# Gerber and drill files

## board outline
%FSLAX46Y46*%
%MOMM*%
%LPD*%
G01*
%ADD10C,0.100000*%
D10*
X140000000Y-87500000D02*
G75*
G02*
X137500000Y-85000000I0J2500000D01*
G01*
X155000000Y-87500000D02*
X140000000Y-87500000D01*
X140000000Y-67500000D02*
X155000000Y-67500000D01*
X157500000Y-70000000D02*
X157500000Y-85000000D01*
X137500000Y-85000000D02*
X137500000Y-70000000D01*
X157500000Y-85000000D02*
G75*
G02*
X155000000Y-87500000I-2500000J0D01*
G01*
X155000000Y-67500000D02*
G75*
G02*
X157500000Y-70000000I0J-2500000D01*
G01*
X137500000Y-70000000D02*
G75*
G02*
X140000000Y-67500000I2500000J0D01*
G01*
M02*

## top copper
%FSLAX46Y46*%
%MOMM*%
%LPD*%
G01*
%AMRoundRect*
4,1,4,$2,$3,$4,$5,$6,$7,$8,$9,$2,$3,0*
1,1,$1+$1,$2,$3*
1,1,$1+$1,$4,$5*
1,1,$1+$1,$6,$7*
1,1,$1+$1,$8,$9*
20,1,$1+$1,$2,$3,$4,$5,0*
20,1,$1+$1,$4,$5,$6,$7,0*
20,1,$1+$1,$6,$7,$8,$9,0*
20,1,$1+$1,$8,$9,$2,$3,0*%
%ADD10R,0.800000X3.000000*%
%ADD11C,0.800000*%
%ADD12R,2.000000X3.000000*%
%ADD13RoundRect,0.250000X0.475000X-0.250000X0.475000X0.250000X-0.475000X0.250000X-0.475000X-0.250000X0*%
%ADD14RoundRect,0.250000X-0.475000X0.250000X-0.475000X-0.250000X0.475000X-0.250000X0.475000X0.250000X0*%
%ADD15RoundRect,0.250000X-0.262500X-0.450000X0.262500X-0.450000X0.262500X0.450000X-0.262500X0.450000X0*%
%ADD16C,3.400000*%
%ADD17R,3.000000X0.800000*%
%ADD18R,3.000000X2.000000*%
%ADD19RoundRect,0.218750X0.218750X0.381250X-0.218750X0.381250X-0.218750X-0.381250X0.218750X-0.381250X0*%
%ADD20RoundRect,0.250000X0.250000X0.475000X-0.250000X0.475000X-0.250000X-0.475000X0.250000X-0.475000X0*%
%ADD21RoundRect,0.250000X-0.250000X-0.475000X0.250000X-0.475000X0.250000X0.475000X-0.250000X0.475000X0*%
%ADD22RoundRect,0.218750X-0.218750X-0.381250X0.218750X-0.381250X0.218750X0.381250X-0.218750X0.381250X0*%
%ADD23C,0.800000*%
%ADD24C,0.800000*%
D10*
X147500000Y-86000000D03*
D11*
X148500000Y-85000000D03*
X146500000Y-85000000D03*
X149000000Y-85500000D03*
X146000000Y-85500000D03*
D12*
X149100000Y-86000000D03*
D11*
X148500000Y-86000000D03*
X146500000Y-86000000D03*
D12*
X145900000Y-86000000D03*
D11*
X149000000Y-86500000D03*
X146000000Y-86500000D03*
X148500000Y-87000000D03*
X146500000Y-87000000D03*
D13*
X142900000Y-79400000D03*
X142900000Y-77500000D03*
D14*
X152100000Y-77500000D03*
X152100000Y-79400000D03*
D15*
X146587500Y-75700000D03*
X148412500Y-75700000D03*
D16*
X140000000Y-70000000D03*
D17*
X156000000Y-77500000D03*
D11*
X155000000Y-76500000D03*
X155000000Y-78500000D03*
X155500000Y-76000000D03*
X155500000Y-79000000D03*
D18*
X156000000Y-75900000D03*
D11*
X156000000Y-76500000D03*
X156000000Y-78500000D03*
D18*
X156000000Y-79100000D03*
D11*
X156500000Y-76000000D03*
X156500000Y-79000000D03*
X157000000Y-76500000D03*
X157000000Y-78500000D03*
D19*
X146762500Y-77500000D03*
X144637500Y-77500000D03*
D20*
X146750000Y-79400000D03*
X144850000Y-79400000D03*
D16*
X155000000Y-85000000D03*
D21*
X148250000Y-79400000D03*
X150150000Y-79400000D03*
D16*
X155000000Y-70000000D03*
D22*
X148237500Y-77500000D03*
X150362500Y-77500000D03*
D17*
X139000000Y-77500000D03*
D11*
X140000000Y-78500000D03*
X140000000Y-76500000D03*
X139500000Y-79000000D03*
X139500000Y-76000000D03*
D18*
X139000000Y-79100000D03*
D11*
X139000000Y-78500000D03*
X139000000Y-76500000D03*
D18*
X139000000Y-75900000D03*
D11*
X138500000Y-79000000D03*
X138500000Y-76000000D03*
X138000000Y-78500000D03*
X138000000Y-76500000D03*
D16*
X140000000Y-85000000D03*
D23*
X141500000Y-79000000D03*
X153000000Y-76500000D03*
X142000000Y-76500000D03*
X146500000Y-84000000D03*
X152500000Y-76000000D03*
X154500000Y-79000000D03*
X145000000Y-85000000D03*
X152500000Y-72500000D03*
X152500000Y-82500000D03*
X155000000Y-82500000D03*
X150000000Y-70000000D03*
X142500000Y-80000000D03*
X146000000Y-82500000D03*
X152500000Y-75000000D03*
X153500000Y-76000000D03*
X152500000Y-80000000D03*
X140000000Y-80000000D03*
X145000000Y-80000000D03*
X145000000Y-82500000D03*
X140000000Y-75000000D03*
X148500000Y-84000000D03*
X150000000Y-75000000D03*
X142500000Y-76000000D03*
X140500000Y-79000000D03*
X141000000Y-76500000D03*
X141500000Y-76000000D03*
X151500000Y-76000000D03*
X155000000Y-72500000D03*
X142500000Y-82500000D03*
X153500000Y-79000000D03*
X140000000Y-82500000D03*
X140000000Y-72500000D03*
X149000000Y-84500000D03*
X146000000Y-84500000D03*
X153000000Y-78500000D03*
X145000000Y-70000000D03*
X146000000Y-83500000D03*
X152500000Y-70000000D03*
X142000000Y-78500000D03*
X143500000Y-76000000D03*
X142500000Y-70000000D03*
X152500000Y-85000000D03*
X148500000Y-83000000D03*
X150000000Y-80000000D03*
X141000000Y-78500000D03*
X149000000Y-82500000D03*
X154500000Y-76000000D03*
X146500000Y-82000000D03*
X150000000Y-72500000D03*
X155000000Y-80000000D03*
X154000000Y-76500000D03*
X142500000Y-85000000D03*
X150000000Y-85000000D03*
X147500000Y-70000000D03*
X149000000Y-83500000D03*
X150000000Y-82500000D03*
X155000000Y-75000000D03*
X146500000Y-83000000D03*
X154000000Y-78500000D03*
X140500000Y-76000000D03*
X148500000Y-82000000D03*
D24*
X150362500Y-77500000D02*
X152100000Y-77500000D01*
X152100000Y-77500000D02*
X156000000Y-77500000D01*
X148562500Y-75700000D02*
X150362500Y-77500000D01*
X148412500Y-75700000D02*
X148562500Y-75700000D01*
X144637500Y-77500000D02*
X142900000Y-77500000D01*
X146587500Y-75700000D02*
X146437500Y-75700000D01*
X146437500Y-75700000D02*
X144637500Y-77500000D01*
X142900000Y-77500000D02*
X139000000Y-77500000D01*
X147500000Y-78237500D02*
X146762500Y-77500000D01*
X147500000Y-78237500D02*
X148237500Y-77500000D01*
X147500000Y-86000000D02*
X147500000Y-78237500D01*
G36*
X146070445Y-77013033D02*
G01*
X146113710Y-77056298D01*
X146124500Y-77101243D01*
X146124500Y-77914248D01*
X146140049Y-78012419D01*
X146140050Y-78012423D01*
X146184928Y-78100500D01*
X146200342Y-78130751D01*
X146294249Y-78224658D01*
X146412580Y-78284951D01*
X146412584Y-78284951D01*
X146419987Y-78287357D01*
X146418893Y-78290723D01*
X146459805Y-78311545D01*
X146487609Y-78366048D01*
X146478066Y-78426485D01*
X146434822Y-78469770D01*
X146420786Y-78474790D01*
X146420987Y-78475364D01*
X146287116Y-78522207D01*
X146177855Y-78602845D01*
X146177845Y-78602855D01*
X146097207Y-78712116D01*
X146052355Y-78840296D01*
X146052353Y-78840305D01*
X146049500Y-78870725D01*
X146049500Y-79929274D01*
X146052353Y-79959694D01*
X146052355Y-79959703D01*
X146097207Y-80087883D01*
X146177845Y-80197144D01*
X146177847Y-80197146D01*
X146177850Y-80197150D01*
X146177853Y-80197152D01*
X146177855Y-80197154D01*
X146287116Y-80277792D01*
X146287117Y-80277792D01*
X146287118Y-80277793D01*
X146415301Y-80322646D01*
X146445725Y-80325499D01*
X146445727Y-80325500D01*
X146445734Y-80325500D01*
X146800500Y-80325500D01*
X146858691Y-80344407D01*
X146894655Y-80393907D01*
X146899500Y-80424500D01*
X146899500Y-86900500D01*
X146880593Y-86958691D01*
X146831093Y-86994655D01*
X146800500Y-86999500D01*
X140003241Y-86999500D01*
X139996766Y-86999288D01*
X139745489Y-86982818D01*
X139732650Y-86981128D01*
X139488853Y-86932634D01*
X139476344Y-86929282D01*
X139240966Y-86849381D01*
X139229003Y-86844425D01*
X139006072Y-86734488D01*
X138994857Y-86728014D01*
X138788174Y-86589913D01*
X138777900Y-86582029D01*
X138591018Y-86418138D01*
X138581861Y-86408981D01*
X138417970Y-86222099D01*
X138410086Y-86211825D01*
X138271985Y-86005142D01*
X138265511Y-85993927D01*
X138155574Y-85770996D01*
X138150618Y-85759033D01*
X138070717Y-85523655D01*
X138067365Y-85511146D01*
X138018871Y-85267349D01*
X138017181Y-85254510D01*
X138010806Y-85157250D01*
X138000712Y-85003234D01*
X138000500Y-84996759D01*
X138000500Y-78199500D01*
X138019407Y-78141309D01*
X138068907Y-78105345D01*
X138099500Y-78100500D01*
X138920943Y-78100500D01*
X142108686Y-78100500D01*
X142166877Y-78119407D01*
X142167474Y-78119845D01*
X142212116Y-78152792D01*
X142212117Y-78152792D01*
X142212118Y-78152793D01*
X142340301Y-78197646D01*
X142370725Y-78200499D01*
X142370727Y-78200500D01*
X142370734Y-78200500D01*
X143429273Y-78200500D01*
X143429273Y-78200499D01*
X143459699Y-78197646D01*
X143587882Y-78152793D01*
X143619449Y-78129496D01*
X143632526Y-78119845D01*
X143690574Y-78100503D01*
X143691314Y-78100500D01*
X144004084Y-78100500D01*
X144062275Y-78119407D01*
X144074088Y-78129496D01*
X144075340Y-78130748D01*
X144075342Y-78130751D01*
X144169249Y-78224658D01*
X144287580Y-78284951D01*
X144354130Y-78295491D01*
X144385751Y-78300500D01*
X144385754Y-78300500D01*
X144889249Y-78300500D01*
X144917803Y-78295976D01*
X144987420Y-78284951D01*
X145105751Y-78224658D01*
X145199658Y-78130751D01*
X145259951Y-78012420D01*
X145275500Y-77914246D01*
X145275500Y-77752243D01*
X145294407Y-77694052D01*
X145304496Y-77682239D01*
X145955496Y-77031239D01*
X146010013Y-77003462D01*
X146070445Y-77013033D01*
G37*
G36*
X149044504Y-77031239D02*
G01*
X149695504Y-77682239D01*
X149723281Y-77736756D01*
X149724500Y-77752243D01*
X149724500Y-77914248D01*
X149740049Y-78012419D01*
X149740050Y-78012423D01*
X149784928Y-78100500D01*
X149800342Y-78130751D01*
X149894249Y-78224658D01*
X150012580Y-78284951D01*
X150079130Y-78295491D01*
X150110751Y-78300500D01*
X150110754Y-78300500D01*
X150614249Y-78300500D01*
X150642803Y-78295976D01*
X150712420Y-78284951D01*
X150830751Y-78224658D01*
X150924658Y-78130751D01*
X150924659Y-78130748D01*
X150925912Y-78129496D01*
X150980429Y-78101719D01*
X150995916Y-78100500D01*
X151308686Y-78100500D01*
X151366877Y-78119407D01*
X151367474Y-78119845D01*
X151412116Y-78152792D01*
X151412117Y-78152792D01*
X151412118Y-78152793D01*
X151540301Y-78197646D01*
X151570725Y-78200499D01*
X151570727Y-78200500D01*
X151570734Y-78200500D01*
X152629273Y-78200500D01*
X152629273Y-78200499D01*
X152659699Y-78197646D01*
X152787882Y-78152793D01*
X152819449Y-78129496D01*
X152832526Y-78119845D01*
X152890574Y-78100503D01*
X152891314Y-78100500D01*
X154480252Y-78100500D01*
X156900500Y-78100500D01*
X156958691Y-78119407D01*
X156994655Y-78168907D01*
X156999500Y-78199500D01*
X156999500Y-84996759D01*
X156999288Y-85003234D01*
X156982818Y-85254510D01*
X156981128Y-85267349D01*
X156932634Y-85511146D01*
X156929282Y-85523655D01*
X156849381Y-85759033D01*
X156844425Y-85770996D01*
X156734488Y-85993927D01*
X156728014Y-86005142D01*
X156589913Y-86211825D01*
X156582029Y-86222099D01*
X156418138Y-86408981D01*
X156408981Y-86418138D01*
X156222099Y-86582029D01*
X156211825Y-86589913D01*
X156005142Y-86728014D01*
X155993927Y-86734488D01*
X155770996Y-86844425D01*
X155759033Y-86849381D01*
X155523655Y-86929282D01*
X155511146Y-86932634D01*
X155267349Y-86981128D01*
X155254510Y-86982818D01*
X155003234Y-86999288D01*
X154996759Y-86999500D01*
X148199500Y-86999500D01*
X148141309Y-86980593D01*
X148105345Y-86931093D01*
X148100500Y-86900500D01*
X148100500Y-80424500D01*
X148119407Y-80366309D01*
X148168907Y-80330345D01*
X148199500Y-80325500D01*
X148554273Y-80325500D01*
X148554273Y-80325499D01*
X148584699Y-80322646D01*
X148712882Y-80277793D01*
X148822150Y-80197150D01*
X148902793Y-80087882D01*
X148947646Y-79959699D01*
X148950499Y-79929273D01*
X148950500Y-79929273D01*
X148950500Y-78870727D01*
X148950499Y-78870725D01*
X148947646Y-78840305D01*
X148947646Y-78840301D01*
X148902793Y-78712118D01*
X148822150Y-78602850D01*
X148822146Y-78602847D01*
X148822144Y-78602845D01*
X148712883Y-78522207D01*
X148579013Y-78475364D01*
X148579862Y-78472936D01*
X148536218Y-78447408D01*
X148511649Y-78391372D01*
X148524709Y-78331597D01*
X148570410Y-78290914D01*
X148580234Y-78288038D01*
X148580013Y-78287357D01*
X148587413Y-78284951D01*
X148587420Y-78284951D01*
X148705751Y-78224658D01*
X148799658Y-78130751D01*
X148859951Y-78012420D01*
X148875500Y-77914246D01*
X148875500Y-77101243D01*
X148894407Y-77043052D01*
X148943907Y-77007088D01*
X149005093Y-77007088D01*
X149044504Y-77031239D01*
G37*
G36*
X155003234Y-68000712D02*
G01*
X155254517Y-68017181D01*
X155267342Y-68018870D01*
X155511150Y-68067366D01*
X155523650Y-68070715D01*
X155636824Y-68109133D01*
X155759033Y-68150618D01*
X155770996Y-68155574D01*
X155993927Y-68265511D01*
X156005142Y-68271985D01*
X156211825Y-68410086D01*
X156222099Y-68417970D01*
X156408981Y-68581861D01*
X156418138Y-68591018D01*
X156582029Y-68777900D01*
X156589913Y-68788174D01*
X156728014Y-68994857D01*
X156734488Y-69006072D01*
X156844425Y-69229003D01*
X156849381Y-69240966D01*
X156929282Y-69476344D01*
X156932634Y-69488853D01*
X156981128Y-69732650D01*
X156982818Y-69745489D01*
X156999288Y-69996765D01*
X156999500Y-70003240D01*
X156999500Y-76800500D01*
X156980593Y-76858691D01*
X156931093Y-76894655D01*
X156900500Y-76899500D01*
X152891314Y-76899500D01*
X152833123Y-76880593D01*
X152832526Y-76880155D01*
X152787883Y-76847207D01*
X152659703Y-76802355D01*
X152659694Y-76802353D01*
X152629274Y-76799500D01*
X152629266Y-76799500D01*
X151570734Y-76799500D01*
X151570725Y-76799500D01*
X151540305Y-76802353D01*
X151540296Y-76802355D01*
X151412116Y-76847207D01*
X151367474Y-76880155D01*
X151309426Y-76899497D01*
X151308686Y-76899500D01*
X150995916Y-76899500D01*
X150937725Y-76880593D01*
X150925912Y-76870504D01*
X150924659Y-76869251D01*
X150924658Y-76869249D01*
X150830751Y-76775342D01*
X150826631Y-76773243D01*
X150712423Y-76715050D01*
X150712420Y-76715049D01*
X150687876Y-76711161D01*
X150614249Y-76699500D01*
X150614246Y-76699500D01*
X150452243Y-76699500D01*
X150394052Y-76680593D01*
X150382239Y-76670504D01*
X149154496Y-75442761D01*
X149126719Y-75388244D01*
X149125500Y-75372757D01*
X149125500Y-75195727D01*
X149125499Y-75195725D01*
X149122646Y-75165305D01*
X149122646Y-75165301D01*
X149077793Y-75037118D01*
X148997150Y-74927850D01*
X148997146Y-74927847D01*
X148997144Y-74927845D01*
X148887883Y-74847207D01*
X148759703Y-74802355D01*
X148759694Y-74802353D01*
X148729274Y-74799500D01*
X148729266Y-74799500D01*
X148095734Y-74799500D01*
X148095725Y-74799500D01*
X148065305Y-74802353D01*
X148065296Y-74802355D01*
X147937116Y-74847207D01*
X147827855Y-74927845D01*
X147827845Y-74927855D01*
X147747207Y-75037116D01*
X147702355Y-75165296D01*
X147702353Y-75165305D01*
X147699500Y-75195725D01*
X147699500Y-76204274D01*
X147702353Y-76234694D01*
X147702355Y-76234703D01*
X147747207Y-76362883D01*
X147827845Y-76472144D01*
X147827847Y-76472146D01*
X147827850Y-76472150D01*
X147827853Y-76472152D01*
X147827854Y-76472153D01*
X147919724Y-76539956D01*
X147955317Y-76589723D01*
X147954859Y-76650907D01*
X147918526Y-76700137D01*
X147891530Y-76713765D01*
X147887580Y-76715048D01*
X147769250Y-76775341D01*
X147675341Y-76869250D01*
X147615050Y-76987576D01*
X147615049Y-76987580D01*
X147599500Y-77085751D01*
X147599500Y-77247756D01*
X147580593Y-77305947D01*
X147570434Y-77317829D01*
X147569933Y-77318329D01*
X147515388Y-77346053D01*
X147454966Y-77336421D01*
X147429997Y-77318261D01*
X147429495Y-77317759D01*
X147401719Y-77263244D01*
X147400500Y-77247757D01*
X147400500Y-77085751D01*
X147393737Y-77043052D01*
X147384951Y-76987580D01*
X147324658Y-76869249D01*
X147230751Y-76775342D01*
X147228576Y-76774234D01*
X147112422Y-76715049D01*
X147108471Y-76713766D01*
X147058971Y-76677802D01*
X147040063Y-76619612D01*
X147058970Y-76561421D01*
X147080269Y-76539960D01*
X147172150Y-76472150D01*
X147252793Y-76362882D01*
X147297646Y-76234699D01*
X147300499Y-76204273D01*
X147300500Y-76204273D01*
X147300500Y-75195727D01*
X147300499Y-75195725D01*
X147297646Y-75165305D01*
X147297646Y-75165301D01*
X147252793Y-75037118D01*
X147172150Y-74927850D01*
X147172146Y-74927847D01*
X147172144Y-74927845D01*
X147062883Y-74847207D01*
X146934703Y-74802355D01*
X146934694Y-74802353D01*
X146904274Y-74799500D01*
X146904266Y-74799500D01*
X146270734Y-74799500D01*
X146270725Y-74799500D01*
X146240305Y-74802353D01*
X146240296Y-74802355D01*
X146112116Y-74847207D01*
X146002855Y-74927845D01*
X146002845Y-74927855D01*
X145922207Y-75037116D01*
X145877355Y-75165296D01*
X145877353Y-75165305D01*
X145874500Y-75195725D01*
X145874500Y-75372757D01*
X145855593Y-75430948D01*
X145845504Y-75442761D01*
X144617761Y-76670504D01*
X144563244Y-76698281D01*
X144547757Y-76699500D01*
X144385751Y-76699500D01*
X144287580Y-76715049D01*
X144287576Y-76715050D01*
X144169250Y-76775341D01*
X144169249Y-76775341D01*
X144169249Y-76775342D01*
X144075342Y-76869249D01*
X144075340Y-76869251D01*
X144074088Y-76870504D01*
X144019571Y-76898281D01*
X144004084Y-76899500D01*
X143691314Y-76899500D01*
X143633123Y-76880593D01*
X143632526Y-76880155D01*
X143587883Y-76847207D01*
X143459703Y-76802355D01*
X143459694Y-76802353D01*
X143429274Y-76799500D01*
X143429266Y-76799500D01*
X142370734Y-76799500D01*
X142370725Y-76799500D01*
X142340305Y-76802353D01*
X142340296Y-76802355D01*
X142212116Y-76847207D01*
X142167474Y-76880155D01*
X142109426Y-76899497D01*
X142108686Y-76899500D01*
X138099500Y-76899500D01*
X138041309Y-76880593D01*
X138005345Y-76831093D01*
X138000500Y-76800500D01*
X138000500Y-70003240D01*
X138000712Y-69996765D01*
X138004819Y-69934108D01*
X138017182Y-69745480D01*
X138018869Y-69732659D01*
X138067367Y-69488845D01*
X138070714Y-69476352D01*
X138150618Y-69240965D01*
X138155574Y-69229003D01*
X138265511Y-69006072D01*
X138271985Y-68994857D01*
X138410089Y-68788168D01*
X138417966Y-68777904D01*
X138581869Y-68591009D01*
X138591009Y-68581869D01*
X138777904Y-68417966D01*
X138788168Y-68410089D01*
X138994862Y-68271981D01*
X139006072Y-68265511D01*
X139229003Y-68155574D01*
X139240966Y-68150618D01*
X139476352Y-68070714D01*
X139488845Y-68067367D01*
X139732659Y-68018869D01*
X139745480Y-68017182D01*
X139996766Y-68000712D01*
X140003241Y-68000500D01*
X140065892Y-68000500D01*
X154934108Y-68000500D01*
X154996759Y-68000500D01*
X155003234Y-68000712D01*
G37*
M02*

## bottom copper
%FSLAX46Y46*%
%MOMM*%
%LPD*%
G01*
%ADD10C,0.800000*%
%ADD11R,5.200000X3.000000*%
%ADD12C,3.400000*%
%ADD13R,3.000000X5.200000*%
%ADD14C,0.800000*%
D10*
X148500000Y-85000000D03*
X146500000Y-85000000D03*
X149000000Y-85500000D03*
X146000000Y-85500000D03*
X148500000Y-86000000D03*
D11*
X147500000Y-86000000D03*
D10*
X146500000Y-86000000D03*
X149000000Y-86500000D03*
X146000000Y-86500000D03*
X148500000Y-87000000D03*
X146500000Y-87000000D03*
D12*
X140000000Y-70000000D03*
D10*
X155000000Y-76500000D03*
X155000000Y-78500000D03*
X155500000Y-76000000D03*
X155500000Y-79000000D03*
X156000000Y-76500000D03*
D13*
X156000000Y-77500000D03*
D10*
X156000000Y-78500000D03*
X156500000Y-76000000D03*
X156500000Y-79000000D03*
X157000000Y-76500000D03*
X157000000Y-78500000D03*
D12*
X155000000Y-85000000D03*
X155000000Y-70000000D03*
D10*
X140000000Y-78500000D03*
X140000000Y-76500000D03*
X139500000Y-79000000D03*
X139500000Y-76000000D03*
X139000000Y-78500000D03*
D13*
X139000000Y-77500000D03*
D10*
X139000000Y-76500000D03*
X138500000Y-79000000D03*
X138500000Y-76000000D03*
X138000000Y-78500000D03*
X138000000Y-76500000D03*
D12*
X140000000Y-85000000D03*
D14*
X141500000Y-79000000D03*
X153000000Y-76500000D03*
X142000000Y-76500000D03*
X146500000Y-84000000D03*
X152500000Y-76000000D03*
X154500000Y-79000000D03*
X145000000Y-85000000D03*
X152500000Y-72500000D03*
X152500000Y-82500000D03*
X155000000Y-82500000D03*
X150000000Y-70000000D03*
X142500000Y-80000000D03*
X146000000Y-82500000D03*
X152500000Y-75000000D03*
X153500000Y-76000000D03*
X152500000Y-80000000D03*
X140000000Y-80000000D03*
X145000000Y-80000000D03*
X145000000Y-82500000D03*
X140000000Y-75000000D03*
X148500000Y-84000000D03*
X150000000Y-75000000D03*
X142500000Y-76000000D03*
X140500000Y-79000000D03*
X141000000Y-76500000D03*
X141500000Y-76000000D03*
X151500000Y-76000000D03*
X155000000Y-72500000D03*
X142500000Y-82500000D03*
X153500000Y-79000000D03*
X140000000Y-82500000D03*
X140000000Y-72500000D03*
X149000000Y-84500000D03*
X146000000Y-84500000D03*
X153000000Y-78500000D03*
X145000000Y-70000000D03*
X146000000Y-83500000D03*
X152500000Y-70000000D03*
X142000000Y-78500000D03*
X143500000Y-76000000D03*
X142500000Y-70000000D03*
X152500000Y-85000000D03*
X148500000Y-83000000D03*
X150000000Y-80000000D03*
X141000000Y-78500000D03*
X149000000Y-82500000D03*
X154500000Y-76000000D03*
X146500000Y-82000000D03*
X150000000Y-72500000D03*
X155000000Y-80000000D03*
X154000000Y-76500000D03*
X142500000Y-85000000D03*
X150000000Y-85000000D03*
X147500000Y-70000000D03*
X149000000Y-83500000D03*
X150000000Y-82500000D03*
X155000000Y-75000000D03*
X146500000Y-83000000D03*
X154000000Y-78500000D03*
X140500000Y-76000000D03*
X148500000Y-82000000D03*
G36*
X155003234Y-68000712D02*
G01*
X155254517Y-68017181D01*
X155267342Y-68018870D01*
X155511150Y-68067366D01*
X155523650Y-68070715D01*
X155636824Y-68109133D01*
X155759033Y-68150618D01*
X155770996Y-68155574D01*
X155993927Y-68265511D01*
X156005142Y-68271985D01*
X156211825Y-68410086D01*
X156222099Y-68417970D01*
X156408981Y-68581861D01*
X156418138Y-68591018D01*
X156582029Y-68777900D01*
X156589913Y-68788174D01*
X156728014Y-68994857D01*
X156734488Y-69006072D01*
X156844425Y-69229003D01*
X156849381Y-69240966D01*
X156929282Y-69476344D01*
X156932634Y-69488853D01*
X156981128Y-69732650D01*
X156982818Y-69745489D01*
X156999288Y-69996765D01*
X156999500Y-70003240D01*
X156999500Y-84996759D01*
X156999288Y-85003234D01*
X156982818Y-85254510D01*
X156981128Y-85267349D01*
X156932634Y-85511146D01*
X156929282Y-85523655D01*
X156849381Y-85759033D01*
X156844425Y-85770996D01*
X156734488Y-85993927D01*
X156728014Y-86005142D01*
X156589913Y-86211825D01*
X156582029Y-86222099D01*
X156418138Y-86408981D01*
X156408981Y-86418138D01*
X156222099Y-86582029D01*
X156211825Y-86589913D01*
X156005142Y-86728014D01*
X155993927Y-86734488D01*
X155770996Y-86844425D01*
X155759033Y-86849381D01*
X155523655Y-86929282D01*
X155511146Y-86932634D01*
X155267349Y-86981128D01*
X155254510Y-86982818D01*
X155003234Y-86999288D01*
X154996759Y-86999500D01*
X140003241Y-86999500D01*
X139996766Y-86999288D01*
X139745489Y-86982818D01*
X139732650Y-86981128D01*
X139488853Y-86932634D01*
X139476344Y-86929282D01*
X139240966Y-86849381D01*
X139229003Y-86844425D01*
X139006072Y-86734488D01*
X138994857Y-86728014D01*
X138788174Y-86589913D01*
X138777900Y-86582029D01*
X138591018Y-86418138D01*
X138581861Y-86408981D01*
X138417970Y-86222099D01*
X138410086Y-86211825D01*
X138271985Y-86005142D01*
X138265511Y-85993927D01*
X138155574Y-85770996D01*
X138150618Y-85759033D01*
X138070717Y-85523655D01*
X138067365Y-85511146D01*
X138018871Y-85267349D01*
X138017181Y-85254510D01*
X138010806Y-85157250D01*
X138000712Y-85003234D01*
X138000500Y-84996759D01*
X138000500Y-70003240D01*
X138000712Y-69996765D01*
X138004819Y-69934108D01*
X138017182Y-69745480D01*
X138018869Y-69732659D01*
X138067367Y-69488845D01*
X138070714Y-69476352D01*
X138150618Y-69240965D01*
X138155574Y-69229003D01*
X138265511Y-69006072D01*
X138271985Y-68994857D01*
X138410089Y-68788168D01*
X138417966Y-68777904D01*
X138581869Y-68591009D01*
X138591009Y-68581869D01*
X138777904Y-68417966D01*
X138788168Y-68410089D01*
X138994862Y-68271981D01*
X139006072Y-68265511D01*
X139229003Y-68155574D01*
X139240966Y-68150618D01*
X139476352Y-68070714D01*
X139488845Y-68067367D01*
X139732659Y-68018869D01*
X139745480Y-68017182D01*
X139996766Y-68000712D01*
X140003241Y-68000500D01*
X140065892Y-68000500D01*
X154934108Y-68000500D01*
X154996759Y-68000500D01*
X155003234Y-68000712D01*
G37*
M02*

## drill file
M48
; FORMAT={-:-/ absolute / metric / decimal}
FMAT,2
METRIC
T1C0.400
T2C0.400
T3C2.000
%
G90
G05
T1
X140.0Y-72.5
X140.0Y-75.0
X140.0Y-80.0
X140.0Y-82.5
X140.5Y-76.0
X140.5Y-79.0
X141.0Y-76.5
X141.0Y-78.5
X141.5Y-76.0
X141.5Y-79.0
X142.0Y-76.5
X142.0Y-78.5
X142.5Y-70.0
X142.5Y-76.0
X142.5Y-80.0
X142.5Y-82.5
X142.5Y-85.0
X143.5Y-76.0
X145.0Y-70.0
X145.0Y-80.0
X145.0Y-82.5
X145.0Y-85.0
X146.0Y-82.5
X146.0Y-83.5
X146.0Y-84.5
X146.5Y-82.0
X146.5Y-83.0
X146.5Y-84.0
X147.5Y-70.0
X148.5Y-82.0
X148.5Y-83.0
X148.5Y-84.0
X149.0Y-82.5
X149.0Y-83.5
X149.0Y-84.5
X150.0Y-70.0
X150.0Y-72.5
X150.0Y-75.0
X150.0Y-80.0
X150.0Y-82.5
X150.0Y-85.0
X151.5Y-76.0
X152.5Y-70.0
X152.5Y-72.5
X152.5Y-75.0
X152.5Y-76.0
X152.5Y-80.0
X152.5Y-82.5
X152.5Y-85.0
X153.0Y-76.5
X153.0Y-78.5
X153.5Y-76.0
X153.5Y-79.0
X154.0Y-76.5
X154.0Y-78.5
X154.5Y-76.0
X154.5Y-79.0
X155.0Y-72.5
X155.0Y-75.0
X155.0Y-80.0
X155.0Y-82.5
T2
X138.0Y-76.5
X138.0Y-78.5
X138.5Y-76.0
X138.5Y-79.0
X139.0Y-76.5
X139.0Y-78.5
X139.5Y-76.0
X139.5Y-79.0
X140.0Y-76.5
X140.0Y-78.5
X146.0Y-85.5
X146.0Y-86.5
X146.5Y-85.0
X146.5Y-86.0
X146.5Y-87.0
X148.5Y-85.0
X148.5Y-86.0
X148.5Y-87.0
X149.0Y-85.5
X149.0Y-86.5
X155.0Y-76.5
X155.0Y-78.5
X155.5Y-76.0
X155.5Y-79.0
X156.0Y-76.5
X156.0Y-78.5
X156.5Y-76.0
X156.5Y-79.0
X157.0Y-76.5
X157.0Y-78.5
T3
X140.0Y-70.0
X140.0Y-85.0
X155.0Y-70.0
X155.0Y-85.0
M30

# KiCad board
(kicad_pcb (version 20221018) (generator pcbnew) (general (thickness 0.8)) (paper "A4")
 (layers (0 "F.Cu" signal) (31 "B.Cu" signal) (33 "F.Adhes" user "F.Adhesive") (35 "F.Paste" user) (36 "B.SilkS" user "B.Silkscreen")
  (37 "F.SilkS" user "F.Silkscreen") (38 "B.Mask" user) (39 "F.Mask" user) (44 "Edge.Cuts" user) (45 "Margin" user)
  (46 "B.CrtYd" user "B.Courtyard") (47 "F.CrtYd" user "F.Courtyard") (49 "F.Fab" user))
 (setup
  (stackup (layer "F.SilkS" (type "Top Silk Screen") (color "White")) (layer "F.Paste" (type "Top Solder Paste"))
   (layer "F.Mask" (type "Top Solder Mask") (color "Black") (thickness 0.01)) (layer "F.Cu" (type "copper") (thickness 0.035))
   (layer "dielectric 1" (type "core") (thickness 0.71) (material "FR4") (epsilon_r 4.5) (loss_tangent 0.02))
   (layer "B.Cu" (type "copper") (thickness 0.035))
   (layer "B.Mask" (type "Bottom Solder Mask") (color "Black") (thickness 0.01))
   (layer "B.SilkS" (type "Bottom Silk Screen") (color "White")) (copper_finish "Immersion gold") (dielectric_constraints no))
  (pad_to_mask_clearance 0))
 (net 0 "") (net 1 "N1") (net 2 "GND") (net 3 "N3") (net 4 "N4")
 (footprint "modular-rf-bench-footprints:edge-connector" (layer "F.Cu") (at 147.5 87.5 -90)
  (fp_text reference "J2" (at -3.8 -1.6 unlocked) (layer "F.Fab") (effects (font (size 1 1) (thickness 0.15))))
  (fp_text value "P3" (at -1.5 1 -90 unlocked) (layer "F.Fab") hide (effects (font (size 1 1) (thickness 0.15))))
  (pad "1" smd rect (at -1.5 0 270) (size 3 0.8) (layers "F.Cu") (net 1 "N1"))
  (pad "2" thru_hole circle (at -2.5 -1 270) (size 0.8 0.8) (drill 0.4) (layers "*.Cu") (remove_unused_layers) (keep_end_layers)
   (zone_layer_connections) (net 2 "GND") (zone_connect 2))
  (pad "2" thru_hole circle (at -2.5 1 270) (size 0.8 0.8) (drill 0.4) (layers "*.Cu") (remove_unused_layers) (keep_end_layers)
   (zone_layer_connections) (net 2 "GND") (zone_connect 2))
  (pad "2" thru_hole circle (at -2 -1.5 270) (size 0.8 0.8) (drill 0.4) (layers "*.Cu") (remove_unused_layers) (keep_end_layers)
   (zone_layer_connections) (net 2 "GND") (zone_connect 2))
  (pad "2" thru_hole circle (at -2 1.5 270) (size 0.8 0.8) (drill 0.4) (layers "*.Cu") (remove_unused_layers) (keep_end_layers)
   (zone_layer_connections) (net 2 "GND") (zone_connect 2))
  (pad "2" smd rect (at -1.5 -1.6 270) (size 3 2) (layers "F.Cu") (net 2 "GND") (zone_connect 2))
  (pad "2" thru_hole circle (at -1.5 -1 270) (size 0.8 0.8) (drill 0.4) (layers "*.Cu") (remove_unused_layers) (keep_end_layers)
   (zone_layer_connections) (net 2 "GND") (zone_connect 2))
  (pad "2" smd rect (at -1.5 0 270) (size 3 5.2) (layers "B.Cu") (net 2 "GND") (zone_connect 2))
  (pad "2" thru_hole circle (at -1.5 1 270) (size 0.8 0.8) (drill 0.4) (layers "*.Cu") (remove_unused_layers) (keep_end_layers)
   (zone_layer_connections) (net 2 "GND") (zone_connect 2))
  (pad "2" smd rect (at -1.5 1.6 270) (size 3 2) (layers "F.Cu") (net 2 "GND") (zone_connect 2))
  (pad "2" thru_hole circle (at -1 -1.5 270) (size 0.8 0.8) (drill 0.4) (layers "*.Cu") (remove_unused_layers) (keep_end_layers)
   (zone_layer_connections) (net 2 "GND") (zone_connect 2))
  (pad "2" thru_hole circle (at -1 1.5 270) (size 0.8 0.8) (drill 0.4) (layers "*.Cu") (remove_unused_layers) (keep_end_layers)
   (zone_layer_connections) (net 2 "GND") (zone_connect 2))
  (pad "2" thru_hole circle (at -0.5 -1 270) (size 0.8 0.8) (drill 0.4) (layers "*.Cu") (remove_unused_layers) (keep_end_layers)
   (zone_layer_connections) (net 2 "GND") (zone_connect 2))
  (pad "2" thru_hole circle (at -0.5 1 270) (size 0.8 0.8) (drill 0.4) (layers "*.Cu") (remove_unused_layers) (keep_end_layers)
   (zone_layer_connections) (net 2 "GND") (zone_connect 2)))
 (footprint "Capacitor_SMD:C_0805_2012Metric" (layer "F.Cu") (at 142.9 78.45 90)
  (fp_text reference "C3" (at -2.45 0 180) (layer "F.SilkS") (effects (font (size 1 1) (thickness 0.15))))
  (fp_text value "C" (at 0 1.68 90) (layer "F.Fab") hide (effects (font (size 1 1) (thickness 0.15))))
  (pad "1" smd roundrect (at -0.95 0 90) (size 1 1.45) (layers "F.Cu" "F.Paste" "F.Mask") (roundrect_rratio 0.25) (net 2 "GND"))
  (pad "2" smd roundrect (at 0.95 0 90) (size 1 1.45) (layers "F.Cu" "F.Paste" "F.Mask") (roundrect_rratio 0.25) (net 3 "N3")))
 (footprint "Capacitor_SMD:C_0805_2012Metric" (layer "F.Cu") (at 152.1 78.45 -90)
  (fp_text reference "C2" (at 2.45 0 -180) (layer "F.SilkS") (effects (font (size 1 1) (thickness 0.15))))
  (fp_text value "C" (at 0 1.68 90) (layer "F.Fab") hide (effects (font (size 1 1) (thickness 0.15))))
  (pad "1" smd roundrect (at -0.95 0 270) (size 1 1.45) (layers "F.Cu" "F.Paste" "F.Mask") (roundrect_rratio 0.25) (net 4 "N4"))
  (pad "2" smd roundrect (at 0.95 0 270) (size 1 1.45) (layers "F.Cu" "F.Paste" "F.Mask") (roundrect_rratio 0.25) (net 2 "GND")))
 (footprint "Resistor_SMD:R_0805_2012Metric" (layer "F.Cu") (at 147.5 75.7)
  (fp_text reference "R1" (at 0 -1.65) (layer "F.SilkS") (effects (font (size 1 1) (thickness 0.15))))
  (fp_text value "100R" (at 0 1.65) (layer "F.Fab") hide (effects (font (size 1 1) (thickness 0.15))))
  (pad "1" smd roundrect (at -0.9125 0) (size 1.025 1.4) (layers "F.Cu" "F.Paste" "F.Mask") (roundrect_rratio 0.243902439) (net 3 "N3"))
  (pad "2" smd roundrect (at 0.9125 0) (size 1.025 1.4) (layers "F.Cu" "F.Paste" "F.Mask") (roundrect_rratio 0.243902439) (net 4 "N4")))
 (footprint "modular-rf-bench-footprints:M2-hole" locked (layer "F.Cu") (at 140 70)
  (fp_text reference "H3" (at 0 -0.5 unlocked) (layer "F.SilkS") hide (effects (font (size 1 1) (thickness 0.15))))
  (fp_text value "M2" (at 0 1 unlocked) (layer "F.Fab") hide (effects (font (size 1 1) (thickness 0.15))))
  (pad "1" thru_hole circle locked (at 0 0) (size 3.4 3.4) (drill 2) (layers "*.Cu" "*.Mask") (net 2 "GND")))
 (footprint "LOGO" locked (layer "F.Cu") (at 144.2 72.5)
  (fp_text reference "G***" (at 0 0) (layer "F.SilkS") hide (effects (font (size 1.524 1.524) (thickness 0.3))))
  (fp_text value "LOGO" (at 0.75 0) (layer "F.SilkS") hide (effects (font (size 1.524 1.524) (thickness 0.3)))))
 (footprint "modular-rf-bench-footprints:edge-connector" (layer "F.Cu") (at 157.5 77.5)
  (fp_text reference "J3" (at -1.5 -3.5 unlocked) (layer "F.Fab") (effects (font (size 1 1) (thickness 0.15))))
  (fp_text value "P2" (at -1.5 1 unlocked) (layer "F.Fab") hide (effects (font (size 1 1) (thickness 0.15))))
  (pad "1" smd rect (at -1.5 0) (size 3 0.8) (layers "F.Cu") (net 4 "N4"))
  (pad "2" thru_hole circle (at -2.5 -1) (size 0.8 0.8) (drill 0.4) (layers "*.Cu") (remove_unused_layers) (keep_end_layers)
   (zone_layer_connections) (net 2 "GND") (zone_connect 2))
  (pad "2" thru_hole circle (at -2.5 1) (size 0.8 0.8) (drill 0.4) (layers "*.Cu") (remove_unused_layers) (keep_end_layers)
   (zone_layer_connections) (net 2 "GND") (zone_connect 2))
  (pad "2" thru_hole circle (at -2 -1.5) (size 0.8 0.8) (drill 0.4) (layers "*.Cu") (remove_unused_layers) (keep_end_layers)
   (zone_layer_connections) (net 2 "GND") (zone_connect 2))
  (pad "2" thru_hole circle (at -2 1.5) (size 0.8 0.8) (drill 0.4) (layers "*.Cu") (remove_unused_layers) (keep_end_layers)
   (zone_layer_connections) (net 2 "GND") (zone_connect 2))
  (pad "2" smd rect (at -1.5 -1.6) (size 3 2) (layers "F.Cu") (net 2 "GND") (zone_connect 2))
  (pad "2" thru_hole circle (at -1.5 -1) (size 0.8 0.8) (drill 0.4) (layers "*.Cu") (remove_unused_layers) (keep_end_layers)
   (zone_layer_connections) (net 2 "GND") (zone_connect 2))
  (pad "2" smd rect (at -1.5 0) (size 3 5.2) (layers "B.Cu") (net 2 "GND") (zone_connect 2))
  (pad "2" thru_hole circle (at -1.5 1) (size 0.8 0.8) (drill 0.4) (layers "*.Cu") (remove_unused_layers) (keep_end_layers)
   (zone_layer_connections) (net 2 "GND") (zone_connect 2))
  (pad "2" smd rect (at -1.5 1.6) (size 3 2) (layers "F.Cu") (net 2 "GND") (zone_connect 2))
  (pad "2" thru_hole circle (at -1 -1.5) (size 0.8 0.8) (drill 0.4) (layers "*.Cu") (remove_unused_layers) (keep_end_layers)
   (zone_layer_connections) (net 2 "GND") (zone_connect 2))
  (pad "2" thru_hole circle (at -1 1.5) (size 0.8 0.8) (drill 0.4) (layers "*.Cu") (remove_unused_layers) (keep_end_layers)
   (zone_layer_connections) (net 2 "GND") (zone_connect 2))
  (pad "2" thru_hole circle (at -0.5 -1) (size 0.8 0.8) (drill 0.4) (layers "*.Cu") (remove_unused_layers) (keep_end_layers)
   (zone_layer_connections) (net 2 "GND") (zone_connect 2))
  (pad "2" thru_hole circle (at -0.5 1) (size 0.8 0.8) (drill 0.4) (layers "*.Cu") (remove_unused_layers) (keep_end_layers)
   (zone_layer_connections) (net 2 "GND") (zone_connect 2)))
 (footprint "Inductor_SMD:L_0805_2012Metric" (layer "F.Cu") (at 145.7 77.5 180)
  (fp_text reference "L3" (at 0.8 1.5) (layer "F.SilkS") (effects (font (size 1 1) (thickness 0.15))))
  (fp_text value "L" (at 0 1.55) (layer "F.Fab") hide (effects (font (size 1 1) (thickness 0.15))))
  (pad "1" smd roundrect (at -1.0625 0 180) (size 0.875 1.2) (layers "F.Cu" "F.Paste" "F.Mask") (roundrect_rratio 0.25) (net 1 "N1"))
  (pad "2" smd roundrect (at 1.0625 0 180) (size 0.875 1.2) (layers "F.Cu" "F.Paste" "F.Mask") (roundrect_rratio 0.25) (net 3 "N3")))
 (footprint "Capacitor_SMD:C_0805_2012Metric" (layer "F.Cu") (at 145.8 79.4 180)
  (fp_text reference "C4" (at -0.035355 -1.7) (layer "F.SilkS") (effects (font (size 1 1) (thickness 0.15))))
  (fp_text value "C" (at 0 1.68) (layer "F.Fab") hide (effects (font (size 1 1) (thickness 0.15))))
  (pad "1" smd roundrect (at -0.95 0 180) (size 1 1.45) (layers "F.Cu" "F.Paste" "F.Mask") (roundrect_rratio 0.25) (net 1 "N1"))
  (pad "2" smd roundrect (at 0.95 0 180) (size 1 1.45) (layers "F.Cu" "F.Paste" "F.Mask") (roundrect_rratio 0.25) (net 2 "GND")))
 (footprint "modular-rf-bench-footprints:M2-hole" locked (layer "F.Cu") (at 155 85)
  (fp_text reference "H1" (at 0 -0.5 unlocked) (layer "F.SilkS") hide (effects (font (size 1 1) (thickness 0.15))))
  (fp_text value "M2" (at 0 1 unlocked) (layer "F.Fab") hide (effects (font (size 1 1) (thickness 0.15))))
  (pad "1" thru_hole circle locked (at 0 0) (size 3.4 3.4) (drill 2) (layers "*.Cu" "*.Mask") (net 2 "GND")))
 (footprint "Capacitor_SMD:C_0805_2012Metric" (layer "F.Cu") (at 149.2 79.4)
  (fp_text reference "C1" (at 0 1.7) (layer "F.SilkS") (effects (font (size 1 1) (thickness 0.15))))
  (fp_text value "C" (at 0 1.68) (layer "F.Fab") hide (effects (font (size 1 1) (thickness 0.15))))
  (pad "1" smd roundrect (at -0.95 0) (size 1 1.45) (layers "F.Cu" "F.Paste" "F.Mask") (roundrect_rratio 0.25) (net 1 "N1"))
  (pad "2" smd roundrect (at 0.95 0) (size 1 1.45) (layers "F.Cu" "F.Paste" "F.Mask") (roundrect_rratio 0.25) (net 2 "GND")))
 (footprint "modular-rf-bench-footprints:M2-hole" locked (layer "F.Cu") (at 155 70)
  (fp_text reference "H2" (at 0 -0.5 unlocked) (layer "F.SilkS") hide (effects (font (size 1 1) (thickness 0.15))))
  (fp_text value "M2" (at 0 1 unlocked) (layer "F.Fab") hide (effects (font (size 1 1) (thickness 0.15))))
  (pad "1" thru_hole circle locked (at 0 0) (size 3.4 3.4) (drill 2) (layers "*.Cu" "*.Mask") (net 2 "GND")))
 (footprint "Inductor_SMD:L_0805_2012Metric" (layer "F.Cu") (at 149.3 77.5)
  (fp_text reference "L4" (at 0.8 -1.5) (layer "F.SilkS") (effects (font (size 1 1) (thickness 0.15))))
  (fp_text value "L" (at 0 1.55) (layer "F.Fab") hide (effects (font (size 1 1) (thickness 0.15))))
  (pad "1" smd roundrect (at -1.0625 0) (size 0.875 1.2) (layers "F.Cu" "F.Paste" "F.Mask") (roundrect_rratio 0.25) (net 1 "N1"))
  (pad "2" smd roundrect (at 1.0625 0) (size 0.875 1.2) (layers "F.Cu" "F.Paste" "F.Mask") (roundrect_rratio 0.25) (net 4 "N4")))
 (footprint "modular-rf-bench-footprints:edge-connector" (layer "F.Cu") (at 137.5 77.5 180)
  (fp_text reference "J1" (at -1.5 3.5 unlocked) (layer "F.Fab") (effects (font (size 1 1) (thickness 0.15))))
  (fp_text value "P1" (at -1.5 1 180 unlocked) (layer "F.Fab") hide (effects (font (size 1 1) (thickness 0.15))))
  (pad "1" smd rect (at -1.5 0 180) (size 3 0.8) (layers "F.Cu") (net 3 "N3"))
  (pad "2" thru_hole circle (at -2.5 -1 180) (size 0.8 0.8) (drill 0.4) (layers "*.Cu") (remove_unused_layers) (keep_end_layers)
   (zone_layer_connections) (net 2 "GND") (zone_connect 2))
  (pad "2" thru_hole circle (at -2.5 1 180) (size 0.8 0.8) (drill 0.4) (layers "*.Cu") (remove_unused_layers) (keep_end_layers)
   (zone_layer_connections) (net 2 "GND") (zone_connect 2))
  (pad "2" thru_hole circle (at -2 -1.5 180) (size 0.8 0.8) (drill 0.4) (layers "*.Cu") (remove_unused_layers) (keep_end_layers)
   (zone_layer_connections) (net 2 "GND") (zone_connect 2))
  (pad "2" thru_hole circle (at -2 1.5 180) (size 0.8 0.8) (drill 0.4) (layers "*.Cu") (remove_unused_layers) (keep_end_layers)
   (zone_layer_connections) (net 2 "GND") (zone_connect 2))
  (pad "2" smd rect (at -1.5 -1.6 180) (size 3 2) (layers "F.Cu") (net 2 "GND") (zone_connect 2))
  (pad "2" thru_hole circle (at -1.5 -1 180) (size 0.8 0.8) (drill 0.4) (layers "*.Cu") (remove_unused_layers) (keep_end_layers)
   (zone_layer_connections) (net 2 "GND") (zone_connect 2))
  (pad "2" smd rect (at -1.5 0 180) (size 3 5.2) (layers "B.Cu") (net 2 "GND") (zone_connect 2))
  (pad "2" thru_hole circle (at -1.5 1 180) (size 0.8 0.8) (drill 0.4) (layers "*.Cu") (remove_unused_layers) (keep_end_layers)
   (zone_layer_connections) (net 2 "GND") (zone_connect 2))
  (pad "2" smd rect (at -1.5 1.6 180) (size 3 2) (layers "F.Cu") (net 2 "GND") (zone_connect 2))
  (pad "2" thru_hole circle (at -1 -1.5 180) (size 0.8 0.8) (drill 0.4) (layers "*.Cu") (remove_unused_layers) (keep_end_layers)
   (zone_layer_connections) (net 2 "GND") (zone_connect 2))
  (pad "2" thru_hole circle (at -1 1.5 180) (size 0.8 0.8) (drill 0.4) (layers "*.Cu") (remove_unused_layers) (keep_end_layers)
   (zone_layer_connections) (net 2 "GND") (zone_connect 2))
  (pad "2" thru_hole circle (at -0.5 -1 180) (size 0.8 0.8) (drill 0.4) (layers "*.Cu") (remove_unused_layers) (keep_end_layers)
   (zone_layer_connections) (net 2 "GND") (zone_connect 2))
  (pad "2" thru_hole circle (at -0.5 1 180) (size 0.8 0.8) (drill 0.4) (layers "*.Cu") (remove_unused_layers) (keep_end_layers)
   (zone_layer_connections) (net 2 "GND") (zone_connect 2)))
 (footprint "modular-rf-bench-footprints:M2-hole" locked (layer "F.Cu") (at 140 85)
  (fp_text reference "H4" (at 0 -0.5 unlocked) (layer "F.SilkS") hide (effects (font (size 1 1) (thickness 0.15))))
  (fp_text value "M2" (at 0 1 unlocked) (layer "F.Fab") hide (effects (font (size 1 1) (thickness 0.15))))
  (pad "1" thru_hole circle locked (at 0 0) (size 3.4 3.4) (drill 2) (layers "*.Cu" "*.Mask") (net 2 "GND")))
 (gr_arc (start 140 87.5) (mid 138.232233 86.767767) (end 137.5 85) (stroke (width 0.1) (type solid)) (layer "Edge.Cuts"))
 (gr_line (start 155 87.5) (end 140 87.5) (stroke (width 0.1) (type solid)) (layer "Edge.Cuts"))
 (gr_line (start 140 67.5) (end 155 67.5) (stroke (width 0.1) (type solid)) (layer "Edge.Cuts"))
 (gr_line (start 157.5 70) (end 157.5 85) (stroke (width 0.1) (type solid)) (layer "Edge.Cuts"))
 (gr_line (start 137.5 85) (end 137.5 70) (stroke (width 0.1) (type solid)) (layer "Edge.Cuts"))
 (gr_arc (start 157.5 85) (mid 156.767767 86.767767) (end 155 87.5) (stroke (width 0.1) (type solid)) (layer "Edge.Cuts"))
 (gr_arc (start 155 67.5) (mid 156.767767 68.232233) (end 157.5 70) (stroke (width 0.1) (type solid)) (layer "Edge.Cuts"))
 (gr_arc (start 137.5 70) (mid 138.232233 68.232233) (end 140 67.5) (stroke (width 0.1) (type solid)) (layer "Edge.Cuts"))
 (via (at 141.5 79) (size 0.8) (drill 0.4) (layers "F.Cu" "B.Cu") (free) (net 2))
 (via (at 153 76.5) (size 0.8) (drill 0.4) (layers "F.Cu" "B.Cu") (free) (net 2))
 (via (at 142 76.5) (size 0.8) (drill 0.4) (layers "F.Cu" "B.Cu") (free) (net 2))
 (via (at 146.5 84) (size 0.8) (drill 0.4) (layers "F.Cu" "B.Cu") (free) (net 2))
 (via (at 152.5 76) (size 0.8) (drill 0.4) (layers "F.Cu" "B.Cu") (free) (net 2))
 (via (at 154.5 79) (size 0.8) (drill 0.4) (layers "F.Cu" "B.Cu") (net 2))
 (via (at 145 85) (size 0.8) (drill 0.4) (layers "F.Cu" "B.Cu") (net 2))
 (via (at 152.5 72.5) (size 0.8) (drill 0.4) (layers "F.Cu" "B.Cu") (free) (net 2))
 (via (at 152.5 82.5) (size 0.8) (drill 0.4) (layers "F.Cu" "B.Cu") (free) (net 2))
 (via (at 155 82.5) (size 0.8) (drill 0.4) (layers "F.Cu" "B.Cu") (free) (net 2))
 (via (at 150 70) (size 0.8) (drill 0.4) (layers "F.Cu" "B.Cu") (free) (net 2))
 (via (at 142.5 80) (size 0.8) (drill 0.4) (layers "F.Cu" "B.Cu") (free) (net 2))
 (via (at 146 82.5) (size 0.8) (drill 0.4) (layers "F.Cu" "B.Cu") (free) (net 2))
 (via (at 152.5 75) (size 0.8) (drill 0.4) (layers "F.Cu" "B.Cu") (free) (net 2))
 (via (at 153.5 76) (size 0.8) (drill 0.4) (layers "F.Cu" "B.Cu") (free) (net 2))
 (via (at 152.5 80) (size 0.8) (drill 0.4) (layers "F.Cu" "B.Cu") (free) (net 2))
 (via (at 140 80) (size 0.8) (drill 0.4) (layers "F.Cu" "B.Cu") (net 2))
 (via (at 145 80) (size 0.8) (drill 0.4) (layers "F.Cu" "B.Cu") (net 2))
 (via (at 145 82.5) (size 0.8) (drill 0.4) (layers "F.Cu" "B.Cu") (free) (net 2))
 (via (at 140 75) (size 0.8) (drill 0.4) (layers "F.Cu" "B.Cu") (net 2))
 (via (at 148.5 84) (size 0.8) (drill 0.4) (layers "F.Cu" "B.Cu") (free) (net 2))
 (via (at 150 75) (size 0.8) (drill 0.4) (layers "F.Cu" "B.Cu") (free) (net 2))
 (via (at 142.5 76) (size 0.8) (drill 0.4) (layers "F.Cu" "B.Cu") (free) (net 2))
 (via (at 140.5 79) (size 0.8) (drill 0.4) (layers "F.Cu" "B.Cu") (free) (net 2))
 (via (at 141 76.5) (size 0.8) (drill 0.4) (layers "F.Cu" "B.Cu") (free) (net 2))
 (via (at 141.5 76) (size 0.8) (drill 0.4) (layers "F.Cu" "B.Cu") (free) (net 2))
 (via (at 151.5 76) (size 0.8) (drill 0.4) (layers "F.Cu" "B.Cu") (free) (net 2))
 (via (at 155 72.5) (size 0.8) (drill 0.4) (layers "F.Cu" "B.Cu") (free) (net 2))
 (via (at 142.5 82.5) (size 0.8) (drill 0.4) (layers "F.Cu" "B.Cu") (free) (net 2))
 (via (at 153.5 79) (size 0.8) (drill 0.4) (layers "F.Cu" "B.Cu") (free) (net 2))
 (via (at 140 82.5) (size 0.8) (drill 0.4) (layers "F.Cu" "B.Cu") (free) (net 2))
 (via (at 140 72.5) (size 0.8) (drill 0.4) (layers "F.Cu" "B.Cu") (free) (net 2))
 (via (at 149 84.5) (size 0.8) (drill 0.4) (layers "F.Cu" "B.Cu") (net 2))
 (via (at 146 84.5) (size 0.8) (drill 0.4) (layers "F.Cu" "B.Cu") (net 2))
 (via (at 153 78.5) (size 0.8) (drill 0.4) (layers "F.Cu" "B.Cu") (free) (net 2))
 (via (at 145 70) (size 0.8) (drill 0.4) (layers "F.Cu" "B.Cu") (free) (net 2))
 (via (at 146 83.5) (size 0.8) (drill 0.4) (layers "F.Cu" "B.Cu") (free) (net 2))
 (via (at 152.5 70) (size 0.8) (drill 0.4) (layers "F.Cu" "B.Cu") (free) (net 2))
 (via (at 142 78.5) (size 0.8) (drill 0.4) (layers "F.Cu" "B.Cu") (free) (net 2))
 (via (at 143.5 76) (size 0.8) (drill 0.4) (layers "F.Cu" "B.Cu") (free) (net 2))
 (via (at 142.5 70) (size 0.8) (drill 0.4) (layers "F.Cu" "B.Cu") (free) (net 2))
 (via (at 152.5 85) (size 0.8) (drill 0.4) (layers "F.Cu" "B.Cu") (free) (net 2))
 (via (at 148.5 83) (size 0.8) (drill 0.4) (layers "F.Cu" "B.Cu") (free) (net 2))
 (via (at 150 80) (size 0.8) (drill 0.4) (layers "F.Cu" "B.Cu") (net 2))
 (via (at 141 78.5) (size 0.8) (drill 0.4) (layers "F.Cu" "B.Cu") (free) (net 2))
 (via (at 149 82.5) (size 0.8) (drill 0.4) (layers "F.Cu" "B.Cu") (free) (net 2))
 (via (at 154.5 76) (size 0.8) (drill 0.4) (layers "F.Cu" "B.Cu") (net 2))
 (via (at 146.5 82) (size 0.8) (drill 0.4) (layers "F.Cu" "B.Cu") (free) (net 2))
 (via (at 150 72.5) (size 0.8) (drill 0.4) (layers "F.Cu" "B.Cu") (free) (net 2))
 (via (at 155 80) (size 0.8) (drill 0.4) (layers "F.Cu" "B.Cu") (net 2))
 (via (at 154 76.5) (size 0.8) (drill 0.4) (layers "F.Cu" "B.Cu") (free) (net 2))
 (via (at 142.5 85) (size 0.8) (drill 0.4) (layers "F.Cu" "B.Cu") (free) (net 2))
 (via (at 150 85) (size 0.8) (drill 0.4) (layers "F.Cu" "B.Cu") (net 2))
 (via (at 147.5 70) (size 0.8) (drill 0.4) (layers "F.Cu" "B.Cu") (free) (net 2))
 (via (at 149 83.5) (size 0.8) (drill 0.4) (layers "F.Cu" "B.Cu") (free) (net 2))
 (via (at 150 82.5) (size 0.8) (drill 0.4) (layers "F.Cu" "B.Cu") (free) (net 2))
 (via (at 155 75) (size 0.8) (drill 0.4) (layers "F.Cu" "B.Cu") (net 2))
 (via (at 146.5 83) (size 0.8) (drill 0.4) (layers "F.Cu" "B.Cu") (free) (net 2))
 (via (at 154 78.5) (size 0.8) (drill 0.4) (layers "F.Cu" "B.Cu") (free) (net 2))
 (via (at 140.5 76) (size 0.8) (drill 0.4) (layers "F.Cu" "B.Cu") (free) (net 2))
 (via (at 148.5 82) (size 0.8) (drill 0.4) (layers "F.Cu" "B.Cu") (free) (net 2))
 (segment (start 150.3625 77.5) (end 152.1 77.5) (width 0.8) (layer "F.Cu") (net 4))
 (segment (start 152.1 77.5) (end 156 77.5) (width 0.8) (layer "F.Cu") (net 4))
 (segment (start 148.5625 75.7) (end 150.3625 77.5) (width 0.8) (layer "F.Cu") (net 4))
 (segment (start 148.4125 75.7) (end 148.5625 75.7) (width 0.8) (layer "F.Cu") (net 4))
 (segment (start 144.6375 77.5) (end 142.9 77.5) (width 0.8) (layer "F.Cu") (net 3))
 (segment (start 146.5875 75.7) (end 146.4375 75.7) (width 0.8) (layer "F.Cu") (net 3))
 (segment (start 146.4375 75.7) (end 144.6375 77.5) (width 0.8) (layer "F.Cu") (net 3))
 (segment (start 142.9 77.5) (end 139 77.5) (width 0.8) (layer "F.Cu") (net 3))
 (segment (start 147.5 78.2375) (end 146.7625 77.5) (width 0.8) (layer "F.Cu") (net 1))
 (segment (start 147.5 78.2375) (end 148.2375 77.5) (width 0.8) (layer "F.Cu") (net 1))
 (segment (start 147.5 86) (end 147.5 78.2375) (width 0.8) (layer "F.Cu") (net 1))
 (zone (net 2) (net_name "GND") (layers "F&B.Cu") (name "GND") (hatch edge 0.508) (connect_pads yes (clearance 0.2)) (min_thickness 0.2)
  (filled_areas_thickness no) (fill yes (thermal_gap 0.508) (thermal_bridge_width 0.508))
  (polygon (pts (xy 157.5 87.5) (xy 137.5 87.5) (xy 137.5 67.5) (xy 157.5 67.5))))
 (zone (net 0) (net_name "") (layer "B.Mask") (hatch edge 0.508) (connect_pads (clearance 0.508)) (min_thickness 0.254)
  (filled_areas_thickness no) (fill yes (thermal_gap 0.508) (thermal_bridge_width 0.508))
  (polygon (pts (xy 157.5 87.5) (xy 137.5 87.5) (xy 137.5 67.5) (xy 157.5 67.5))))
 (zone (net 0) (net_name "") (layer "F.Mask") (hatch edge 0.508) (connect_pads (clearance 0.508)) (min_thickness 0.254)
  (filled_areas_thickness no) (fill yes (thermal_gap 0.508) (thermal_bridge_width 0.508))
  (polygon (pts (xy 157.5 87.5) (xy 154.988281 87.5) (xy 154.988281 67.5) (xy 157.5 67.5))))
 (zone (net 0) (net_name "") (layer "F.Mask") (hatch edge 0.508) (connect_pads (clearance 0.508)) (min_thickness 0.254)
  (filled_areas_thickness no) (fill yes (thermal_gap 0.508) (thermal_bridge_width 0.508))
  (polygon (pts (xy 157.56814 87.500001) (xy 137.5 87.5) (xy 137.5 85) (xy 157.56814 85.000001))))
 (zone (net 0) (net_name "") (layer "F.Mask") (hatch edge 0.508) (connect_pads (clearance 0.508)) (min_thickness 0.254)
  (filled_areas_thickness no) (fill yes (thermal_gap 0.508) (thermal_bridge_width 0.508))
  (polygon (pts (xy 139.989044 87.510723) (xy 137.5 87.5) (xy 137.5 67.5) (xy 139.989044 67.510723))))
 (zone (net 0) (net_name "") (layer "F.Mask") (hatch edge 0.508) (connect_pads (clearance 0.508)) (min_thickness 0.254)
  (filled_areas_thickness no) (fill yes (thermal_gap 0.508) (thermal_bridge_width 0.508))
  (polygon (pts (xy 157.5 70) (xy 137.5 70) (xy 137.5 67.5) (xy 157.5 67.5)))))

